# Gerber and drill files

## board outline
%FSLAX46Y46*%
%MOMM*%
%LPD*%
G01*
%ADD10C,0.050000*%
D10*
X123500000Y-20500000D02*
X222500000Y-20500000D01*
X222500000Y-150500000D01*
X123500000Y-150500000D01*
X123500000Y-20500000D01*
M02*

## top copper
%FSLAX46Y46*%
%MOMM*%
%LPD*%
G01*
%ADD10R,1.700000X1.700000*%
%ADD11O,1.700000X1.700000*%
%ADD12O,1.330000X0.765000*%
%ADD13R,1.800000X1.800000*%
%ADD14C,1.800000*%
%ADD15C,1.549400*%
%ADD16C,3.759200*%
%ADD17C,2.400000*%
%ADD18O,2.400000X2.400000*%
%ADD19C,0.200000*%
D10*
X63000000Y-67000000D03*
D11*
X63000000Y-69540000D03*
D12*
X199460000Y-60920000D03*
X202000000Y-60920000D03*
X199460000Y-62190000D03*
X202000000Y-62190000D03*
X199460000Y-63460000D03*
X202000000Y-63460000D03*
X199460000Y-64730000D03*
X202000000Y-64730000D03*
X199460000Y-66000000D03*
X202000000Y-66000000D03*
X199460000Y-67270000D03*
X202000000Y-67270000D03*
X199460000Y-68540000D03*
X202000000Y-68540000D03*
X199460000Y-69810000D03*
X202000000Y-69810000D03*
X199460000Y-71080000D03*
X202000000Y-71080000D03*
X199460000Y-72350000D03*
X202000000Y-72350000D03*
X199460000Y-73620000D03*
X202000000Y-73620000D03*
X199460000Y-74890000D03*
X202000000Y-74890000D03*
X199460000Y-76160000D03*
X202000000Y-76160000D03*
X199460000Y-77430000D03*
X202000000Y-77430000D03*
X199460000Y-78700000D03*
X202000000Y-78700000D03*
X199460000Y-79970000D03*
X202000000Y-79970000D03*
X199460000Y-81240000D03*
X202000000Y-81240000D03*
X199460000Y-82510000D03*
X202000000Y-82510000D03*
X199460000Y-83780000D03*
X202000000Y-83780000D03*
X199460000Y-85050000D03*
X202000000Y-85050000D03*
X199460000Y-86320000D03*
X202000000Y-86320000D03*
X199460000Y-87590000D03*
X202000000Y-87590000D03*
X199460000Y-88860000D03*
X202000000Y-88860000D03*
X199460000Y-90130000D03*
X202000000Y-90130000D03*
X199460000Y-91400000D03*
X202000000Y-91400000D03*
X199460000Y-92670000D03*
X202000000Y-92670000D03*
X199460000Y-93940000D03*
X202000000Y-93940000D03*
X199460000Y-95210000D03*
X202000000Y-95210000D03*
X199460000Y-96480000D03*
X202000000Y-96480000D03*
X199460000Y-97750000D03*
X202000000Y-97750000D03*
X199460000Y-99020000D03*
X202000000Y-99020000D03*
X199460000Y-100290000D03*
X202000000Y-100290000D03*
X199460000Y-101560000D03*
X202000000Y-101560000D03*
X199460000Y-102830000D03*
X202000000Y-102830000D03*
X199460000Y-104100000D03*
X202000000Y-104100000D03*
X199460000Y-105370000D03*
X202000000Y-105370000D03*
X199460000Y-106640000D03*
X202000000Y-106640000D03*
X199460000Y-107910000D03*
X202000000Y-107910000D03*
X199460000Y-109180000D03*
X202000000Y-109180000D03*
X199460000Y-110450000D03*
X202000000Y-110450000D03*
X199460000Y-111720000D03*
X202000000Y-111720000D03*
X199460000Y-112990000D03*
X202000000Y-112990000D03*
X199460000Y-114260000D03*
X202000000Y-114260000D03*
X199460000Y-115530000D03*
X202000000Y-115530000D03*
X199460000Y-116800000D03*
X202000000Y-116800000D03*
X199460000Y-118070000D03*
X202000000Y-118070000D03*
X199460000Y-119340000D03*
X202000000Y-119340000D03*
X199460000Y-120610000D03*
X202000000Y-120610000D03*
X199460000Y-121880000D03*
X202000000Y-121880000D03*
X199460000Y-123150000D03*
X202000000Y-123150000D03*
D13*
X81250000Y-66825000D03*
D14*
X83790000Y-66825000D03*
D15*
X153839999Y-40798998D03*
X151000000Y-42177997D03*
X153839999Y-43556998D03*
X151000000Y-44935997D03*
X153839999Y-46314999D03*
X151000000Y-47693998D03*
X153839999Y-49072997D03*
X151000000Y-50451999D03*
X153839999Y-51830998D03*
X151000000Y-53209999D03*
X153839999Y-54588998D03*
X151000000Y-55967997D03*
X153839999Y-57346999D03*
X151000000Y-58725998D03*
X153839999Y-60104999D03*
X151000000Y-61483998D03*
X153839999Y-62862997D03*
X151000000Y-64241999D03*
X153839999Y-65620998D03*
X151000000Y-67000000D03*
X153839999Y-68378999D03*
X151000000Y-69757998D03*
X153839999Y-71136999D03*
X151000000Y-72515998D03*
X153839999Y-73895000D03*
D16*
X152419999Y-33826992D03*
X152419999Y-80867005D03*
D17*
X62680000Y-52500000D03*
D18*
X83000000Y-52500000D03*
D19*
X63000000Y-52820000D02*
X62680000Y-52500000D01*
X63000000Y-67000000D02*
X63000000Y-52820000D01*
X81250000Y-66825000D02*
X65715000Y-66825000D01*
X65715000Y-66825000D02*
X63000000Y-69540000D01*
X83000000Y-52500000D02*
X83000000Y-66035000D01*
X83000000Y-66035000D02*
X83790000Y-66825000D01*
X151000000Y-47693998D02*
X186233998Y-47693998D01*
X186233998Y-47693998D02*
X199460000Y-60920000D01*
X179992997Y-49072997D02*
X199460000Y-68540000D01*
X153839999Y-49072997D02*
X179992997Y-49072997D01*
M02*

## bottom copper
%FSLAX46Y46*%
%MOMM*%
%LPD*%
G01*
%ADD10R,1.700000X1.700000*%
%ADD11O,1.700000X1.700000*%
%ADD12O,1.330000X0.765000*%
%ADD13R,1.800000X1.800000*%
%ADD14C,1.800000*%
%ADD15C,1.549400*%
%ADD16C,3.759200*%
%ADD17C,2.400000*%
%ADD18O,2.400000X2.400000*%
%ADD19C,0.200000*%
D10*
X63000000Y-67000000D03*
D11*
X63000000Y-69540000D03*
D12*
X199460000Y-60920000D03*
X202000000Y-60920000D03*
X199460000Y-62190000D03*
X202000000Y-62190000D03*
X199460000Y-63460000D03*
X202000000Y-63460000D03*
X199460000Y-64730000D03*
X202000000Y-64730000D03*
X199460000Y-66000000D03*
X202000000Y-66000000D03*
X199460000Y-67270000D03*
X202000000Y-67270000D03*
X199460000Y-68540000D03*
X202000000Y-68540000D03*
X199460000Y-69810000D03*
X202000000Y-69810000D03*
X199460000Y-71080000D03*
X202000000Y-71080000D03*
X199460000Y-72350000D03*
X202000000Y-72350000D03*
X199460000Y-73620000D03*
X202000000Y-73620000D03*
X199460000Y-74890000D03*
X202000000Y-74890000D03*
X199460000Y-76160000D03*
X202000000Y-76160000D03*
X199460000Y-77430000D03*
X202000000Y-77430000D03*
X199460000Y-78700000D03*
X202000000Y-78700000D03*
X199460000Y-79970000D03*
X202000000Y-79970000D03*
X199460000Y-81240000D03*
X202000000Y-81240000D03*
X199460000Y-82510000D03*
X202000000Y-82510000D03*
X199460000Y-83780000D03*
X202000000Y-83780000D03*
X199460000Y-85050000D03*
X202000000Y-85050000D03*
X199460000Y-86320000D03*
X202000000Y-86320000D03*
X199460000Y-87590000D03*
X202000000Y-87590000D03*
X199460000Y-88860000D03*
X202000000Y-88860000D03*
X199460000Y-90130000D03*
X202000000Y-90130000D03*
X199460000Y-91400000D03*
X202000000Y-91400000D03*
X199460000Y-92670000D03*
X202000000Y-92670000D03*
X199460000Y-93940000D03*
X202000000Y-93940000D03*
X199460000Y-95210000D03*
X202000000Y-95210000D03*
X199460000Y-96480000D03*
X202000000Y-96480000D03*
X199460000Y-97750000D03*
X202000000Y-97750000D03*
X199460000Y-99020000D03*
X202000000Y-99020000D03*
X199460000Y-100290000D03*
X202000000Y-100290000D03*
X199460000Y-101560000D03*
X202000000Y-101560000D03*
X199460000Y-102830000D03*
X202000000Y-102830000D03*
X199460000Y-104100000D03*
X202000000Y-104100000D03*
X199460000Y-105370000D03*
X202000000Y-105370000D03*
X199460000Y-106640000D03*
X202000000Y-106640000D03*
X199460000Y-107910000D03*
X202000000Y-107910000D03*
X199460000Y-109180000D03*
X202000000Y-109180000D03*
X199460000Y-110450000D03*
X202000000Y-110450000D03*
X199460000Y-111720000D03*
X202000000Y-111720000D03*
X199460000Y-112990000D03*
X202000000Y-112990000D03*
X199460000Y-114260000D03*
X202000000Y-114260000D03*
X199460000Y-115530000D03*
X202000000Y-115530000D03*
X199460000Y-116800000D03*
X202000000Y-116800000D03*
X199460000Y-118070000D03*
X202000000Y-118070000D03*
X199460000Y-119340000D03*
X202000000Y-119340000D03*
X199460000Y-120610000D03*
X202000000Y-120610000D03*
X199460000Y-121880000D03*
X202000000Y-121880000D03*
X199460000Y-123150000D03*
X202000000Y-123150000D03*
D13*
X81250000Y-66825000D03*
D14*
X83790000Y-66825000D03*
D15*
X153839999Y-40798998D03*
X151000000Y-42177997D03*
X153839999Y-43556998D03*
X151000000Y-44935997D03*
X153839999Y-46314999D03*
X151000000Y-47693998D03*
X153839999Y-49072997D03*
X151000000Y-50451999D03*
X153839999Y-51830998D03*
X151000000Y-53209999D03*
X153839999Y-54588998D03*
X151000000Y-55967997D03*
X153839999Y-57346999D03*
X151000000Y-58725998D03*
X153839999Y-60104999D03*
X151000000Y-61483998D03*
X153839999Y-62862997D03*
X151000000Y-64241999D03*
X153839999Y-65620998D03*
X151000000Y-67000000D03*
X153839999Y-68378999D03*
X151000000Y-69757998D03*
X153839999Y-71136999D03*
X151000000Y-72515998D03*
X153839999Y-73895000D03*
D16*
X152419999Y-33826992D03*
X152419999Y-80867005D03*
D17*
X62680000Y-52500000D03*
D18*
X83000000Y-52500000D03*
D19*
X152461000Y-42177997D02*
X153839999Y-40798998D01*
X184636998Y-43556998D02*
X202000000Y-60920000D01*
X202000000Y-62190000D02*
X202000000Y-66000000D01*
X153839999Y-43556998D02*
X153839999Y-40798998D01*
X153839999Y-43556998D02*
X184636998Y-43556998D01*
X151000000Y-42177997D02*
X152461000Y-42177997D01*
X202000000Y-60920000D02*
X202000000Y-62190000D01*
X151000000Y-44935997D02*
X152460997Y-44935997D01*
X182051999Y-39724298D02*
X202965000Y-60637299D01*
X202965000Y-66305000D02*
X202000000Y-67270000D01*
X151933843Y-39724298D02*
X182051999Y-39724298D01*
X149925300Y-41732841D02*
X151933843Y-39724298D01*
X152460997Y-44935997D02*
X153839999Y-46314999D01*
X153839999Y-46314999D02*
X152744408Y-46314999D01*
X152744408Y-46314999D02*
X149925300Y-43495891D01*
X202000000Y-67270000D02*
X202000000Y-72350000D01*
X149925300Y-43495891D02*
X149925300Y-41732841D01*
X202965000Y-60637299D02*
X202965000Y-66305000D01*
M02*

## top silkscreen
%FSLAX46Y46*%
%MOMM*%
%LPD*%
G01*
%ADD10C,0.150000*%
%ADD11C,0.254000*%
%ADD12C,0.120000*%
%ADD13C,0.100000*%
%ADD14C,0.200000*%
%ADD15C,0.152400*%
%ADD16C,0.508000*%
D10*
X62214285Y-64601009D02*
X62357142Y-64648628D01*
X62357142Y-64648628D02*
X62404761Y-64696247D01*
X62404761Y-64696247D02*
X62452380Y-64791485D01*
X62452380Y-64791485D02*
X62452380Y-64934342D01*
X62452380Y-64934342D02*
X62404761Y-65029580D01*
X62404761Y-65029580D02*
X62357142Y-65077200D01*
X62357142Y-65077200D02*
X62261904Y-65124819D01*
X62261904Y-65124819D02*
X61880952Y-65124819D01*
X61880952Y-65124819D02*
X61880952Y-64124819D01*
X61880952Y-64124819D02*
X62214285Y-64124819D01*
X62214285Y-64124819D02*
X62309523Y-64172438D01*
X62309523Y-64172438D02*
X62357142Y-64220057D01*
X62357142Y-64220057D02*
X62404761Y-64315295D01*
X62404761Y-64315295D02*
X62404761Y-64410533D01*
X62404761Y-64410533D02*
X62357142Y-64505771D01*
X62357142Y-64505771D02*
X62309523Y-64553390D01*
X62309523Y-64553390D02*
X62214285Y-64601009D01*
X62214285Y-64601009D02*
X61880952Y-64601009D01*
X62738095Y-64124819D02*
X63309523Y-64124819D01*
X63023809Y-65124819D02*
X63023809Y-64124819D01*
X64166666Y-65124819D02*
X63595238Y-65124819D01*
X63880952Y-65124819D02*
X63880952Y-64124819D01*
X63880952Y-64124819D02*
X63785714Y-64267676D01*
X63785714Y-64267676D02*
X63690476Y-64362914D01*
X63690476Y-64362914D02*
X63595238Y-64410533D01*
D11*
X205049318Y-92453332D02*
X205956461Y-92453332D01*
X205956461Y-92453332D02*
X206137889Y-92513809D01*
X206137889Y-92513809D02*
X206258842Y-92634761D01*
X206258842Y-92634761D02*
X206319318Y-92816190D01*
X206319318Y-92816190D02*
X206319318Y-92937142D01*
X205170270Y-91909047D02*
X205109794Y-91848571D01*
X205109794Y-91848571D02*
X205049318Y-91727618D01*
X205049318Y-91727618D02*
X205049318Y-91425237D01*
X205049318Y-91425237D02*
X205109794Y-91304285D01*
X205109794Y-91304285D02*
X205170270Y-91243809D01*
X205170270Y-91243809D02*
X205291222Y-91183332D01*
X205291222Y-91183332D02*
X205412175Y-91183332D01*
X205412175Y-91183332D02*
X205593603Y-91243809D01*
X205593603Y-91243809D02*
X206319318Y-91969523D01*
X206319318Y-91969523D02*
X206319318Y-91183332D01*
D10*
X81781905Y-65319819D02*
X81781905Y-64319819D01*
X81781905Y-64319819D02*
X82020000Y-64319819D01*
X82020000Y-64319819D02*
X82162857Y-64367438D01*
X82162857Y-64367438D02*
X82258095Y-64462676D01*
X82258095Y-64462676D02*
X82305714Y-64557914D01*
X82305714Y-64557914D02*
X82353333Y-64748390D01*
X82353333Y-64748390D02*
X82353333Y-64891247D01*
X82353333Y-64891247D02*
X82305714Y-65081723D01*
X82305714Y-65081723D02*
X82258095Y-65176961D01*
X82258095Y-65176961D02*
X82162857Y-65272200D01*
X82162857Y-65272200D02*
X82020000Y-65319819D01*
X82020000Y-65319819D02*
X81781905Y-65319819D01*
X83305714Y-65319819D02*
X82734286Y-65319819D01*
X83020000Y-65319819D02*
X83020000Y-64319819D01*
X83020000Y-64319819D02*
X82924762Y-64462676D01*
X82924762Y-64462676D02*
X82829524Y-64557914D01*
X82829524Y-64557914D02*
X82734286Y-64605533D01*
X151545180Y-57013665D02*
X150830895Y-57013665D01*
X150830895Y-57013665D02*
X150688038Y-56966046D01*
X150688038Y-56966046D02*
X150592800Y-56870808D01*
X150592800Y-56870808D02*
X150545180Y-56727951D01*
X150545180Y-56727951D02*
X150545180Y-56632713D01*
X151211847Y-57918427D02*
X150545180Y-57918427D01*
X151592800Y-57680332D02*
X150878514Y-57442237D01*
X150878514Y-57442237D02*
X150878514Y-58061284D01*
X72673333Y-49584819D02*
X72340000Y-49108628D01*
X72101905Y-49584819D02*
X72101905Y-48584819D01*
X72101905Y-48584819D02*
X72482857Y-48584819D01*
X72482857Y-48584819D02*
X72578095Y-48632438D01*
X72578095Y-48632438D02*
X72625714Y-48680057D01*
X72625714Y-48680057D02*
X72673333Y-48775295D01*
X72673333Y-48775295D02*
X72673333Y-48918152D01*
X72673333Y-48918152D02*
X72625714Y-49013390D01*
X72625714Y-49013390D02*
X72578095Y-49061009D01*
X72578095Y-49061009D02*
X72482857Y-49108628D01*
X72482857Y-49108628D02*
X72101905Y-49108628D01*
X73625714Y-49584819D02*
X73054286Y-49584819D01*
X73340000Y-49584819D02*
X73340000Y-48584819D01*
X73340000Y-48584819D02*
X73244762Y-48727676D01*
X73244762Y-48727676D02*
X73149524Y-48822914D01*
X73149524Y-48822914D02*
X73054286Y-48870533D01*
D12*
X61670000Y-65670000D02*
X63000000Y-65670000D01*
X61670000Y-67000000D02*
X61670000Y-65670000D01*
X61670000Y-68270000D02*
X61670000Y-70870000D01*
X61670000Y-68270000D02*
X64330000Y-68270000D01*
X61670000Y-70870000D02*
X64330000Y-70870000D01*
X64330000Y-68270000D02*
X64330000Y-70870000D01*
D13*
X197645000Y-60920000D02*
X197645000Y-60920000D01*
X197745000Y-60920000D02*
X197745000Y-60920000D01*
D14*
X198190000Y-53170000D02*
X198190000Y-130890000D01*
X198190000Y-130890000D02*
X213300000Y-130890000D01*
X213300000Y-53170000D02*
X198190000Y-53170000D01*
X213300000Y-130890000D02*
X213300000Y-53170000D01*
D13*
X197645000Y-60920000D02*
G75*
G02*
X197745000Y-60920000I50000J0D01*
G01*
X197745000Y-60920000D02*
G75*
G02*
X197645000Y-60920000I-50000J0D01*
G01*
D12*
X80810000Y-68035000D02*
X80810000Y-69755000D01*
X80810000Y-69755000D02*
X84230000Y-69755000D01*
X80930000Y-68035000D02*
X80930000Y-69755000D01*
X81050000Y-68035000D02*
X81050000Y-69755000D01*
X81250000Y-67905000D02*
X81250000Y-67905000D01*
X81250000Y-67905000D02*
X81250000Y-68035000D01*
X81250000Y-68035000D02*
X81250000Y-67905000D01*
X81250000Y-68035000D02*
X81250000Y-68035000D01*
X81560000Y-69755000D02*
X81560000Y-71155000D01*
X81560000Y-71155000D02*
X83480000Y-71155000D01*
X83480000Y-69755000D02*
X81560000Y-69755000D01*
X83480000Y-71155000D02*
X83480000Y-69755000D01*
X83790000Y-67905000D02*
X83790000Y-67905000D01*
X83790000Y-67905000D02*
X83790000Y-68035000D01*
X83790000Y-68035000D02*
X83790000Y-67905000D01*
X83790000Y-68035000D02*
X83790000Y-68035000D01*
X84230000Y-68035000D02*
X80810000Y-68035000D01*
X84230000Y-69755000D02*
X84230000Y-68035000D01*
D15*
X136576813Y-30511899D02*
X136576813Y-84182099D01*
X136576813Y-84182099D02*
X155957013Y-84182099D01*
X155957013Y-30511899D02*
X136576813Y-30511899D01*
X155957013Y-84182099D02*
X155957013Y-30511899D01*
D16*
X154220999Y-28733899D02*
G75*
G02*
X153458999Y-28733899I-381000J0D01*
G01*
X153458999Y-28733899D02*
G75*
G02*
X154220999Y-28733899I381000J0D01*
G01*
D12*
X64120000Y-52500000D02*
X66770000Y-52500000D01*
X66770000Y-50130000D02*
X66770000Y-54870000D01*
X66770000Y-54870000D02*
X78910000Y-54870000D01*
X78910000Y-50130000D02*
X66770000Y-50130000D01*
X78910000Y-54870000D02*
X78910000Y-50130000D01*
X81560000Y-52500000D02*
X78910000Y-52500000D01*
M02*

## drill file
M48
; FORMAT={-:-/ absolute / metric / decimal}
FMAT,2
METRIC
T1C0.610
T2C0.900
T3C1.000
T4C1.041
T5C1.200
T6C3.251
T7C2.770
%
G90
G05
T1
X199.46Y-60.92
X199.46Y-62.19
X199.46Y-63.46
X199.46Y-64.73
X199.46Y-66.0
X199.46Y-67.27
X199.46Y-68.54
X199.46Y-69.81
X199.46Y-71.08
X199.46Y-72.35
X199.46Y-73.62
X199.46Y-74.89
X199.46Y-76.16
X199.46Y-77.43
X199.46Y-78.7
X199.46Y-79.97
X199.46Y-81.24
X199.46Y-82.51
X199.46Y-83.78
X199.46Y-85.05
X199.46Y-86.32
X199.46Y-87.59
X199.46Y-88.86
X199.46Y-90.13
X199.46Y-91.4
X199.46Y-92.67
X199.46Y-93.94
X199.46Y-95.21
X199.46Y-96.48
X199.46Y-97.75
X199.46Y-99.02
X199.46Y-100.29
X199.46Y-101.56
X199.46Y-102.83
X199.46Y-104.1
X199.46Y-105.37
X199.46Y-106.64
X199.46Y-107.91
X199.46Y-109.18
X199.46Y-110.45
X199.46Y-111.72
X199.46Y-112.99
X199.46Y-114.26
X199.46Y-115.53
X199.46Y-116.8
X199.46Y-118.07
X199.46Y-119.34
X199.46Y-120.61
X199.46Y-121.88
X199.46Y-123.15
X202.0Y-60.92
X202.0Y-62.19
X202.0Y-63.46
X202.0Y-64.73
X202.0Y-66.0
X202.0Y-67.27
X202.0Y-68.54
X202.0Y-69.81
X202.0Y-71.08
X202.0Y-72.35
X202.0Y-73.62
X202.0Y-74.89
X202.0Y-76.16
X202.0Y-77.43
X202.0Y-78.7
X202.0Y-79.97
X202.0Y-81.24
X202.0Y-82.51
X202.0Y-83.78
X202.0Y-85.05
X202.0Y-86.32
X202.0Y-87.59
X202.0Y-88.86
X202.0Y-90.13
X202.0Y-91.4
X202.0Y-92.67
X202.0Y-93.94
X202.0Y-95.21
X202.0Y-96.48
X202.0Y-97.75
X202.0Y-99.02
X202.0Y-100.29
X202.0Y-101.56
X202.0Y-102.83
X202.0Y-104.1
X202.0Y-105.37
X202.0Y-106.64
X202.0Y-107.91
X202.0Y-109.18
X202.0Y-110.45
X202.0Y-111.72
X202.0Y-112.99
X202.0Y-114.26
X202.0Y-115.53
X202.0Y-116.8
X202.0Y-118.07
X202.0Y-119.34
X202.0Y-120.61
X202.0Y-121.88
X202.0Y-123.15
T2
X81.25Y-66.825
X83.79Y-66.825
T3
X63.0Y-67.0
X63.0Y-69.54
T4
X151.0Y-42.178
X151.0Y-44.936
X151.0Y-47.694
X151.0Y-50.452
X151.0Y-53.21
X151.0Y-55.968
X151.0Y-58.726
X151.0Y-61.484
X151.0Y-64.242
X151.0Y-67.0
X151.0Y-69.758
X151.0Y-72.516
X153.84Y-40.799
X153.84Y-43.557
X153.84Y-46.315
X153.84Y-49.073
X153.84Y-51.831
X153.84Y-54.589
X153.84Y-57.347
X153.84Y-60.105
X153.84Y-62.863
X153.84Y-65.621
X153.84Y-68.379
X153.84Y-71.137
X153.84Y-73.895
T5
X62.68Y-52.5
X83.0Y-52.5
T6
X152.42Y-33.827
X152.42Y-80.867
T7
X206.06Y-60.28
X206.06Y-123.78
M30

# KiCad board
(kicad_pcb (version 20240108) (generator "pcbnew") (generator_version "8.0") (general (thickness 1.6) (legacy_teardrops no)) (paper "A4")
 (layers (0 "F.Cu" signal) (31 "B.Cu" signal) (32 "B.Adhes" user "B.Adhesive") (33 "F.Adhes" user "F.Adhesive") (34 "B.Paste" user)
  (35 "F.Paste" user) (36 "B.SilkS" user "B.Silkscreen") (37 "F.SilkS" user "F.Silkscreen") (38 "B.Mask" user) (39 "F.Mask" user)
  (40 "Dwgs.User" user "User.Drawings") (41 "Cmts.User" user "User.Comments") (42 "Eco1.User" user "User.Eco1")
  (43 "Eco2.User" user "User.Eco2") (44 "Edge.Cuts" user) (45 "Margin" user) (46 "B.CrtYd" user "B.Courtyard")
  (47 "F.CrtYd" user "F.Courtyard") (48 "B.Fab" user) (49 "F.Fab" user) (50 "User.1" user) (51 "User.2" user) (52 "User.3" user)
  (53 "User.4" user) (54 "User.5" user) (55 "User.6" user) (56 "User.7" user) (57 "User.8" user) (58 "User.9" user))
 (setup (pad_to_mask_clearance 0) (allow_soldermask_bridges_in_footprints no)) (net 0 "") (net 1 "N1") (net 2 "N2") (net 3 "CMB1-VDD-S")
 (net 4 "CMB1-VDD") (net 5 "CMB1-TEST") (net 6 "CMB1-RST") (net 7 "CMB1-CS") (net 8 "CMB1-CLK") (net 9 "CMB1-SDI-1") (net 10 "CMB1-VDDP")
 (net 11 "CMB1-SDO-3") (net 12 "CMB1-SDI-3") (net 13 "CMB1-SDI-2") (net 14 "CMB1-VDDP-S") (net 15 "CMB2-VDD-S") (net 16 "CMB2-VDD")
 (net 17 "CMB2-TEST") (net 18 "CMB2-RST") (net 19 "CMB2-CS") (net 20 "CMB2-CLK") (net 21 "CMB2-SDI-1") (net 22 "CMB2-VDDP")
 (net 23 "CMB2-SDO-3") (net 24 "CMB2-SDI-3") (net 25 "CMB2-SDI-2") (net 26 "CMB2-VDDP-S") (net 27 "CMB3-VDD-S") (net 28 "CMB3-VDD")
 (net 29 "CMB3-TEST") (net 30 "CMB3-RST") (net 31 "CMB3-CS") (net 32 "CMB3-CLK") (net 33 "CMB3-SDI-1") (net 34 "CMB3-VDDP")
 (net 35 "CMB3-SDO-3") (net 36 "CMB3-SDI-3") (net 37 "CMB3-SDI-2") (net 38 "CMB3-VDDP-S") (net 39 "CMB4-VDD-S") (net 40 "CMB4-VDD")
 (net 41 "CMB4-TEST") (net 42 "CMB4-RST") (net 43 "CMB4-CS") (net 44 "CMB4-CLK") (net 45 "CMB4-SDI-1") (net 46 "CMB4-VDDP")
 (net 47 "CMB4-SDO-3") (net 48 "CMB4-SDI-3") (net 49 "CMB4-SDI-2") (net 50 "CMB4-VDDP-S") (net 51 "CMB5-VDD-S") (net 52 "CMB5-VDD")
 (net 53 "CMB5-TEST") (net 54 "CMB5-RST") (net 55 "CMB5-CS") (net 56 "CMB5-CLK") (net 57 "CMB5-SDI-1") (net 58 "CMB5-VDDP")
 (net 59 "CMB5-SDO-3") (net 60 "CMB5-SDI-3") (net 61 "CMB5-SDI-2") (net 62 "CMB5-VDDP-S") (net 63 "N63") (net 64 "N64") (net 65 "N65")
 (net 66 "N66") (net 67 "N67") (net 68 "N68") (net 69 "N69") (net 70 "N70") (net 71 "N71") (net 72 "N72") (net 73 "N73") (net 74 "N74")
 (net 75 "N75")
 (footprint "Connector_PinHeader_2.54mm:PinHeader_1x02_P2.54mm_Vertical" (layer "F.Cu") (at 63 67)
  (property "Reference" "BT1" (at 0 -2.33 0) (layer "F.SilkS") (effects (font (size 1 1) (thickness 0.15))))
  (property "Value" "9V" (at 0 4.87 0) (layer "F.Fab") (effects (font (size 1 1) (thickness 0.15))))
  (fp_line (start -1.33 -1.33) (end 0 -1.33) (stroke (width 0.12) (type solid)) (layer "F.SilkS"))
  (fp_line (start -1.33 0) (end -1.33 -1.33) (stroke (width 0.12) (type solid)) (layer "F.SilkS"))
  (fp_line (start -1.33 1.27) (end -1.33 3.87) (stroke (width 0.12) (type solid)) (layer "F.SilkS"))
  (fp_line (start -1.33 1.27) (end 1.33 1.27) (stroke (width 0.12) (type solid)) (layer "F.SilkS"))
  (fp_line (start -1.33 3.87) (end 1.33 3.87) (stroke (width 0.12) (type solid)) (layer "F.SilkS"))
  (fp_line (start 1.33 1.27) (end 1.33 3.87) (stroke (width 0.12) (type solid)) (layer "F.SilkS"))
  (pad "1" thru_hole rect (at 0 0) (size 1.7 1.7) (drill 1) (layers "*.Cu" "*.Mask") (remove_unused_layers no) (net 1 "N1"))
  (pad "2" thru_hole oval (at 0 2.54) (size 1.7 1.7) (drill 1) (layers "*.Cu" "*.Mask") (remove_unused_layers no) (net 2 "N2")))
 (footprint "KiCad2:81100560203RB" (layer "F.Cu") (at 199.46 60.92 -90)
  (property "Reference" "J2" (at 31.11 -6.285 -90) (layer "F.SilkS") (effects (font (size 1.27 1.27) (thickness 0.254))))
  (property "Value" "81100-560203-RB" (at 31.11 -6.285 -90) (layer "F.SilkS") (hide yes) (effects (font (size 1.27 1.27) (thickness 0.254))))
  (fp_line (start 0 1.815) (end 0 1.815) (stroke (width 0.1) (type solid)) (layer "F.SilkS"))
  (fp_line (start 0 1.715) (end 0 1.715) (stroke (width 0.1) (type solid)) (layer "F.SilkS"))
  (fp_line (start -7.75 1.27) (end 69.97 1.27) (stroke (width 0.2) (type solid)) (layer "F.SilkS"))
  (fp_line (start 69.97 1.27) (end 69.97 -13.84) (stroke (width 0.2) (type solid)) (layer "F.SilkS"))
  (fp_line (start -7.75 -13.84) (end -7.75 1.27) (stroke (width 0.2) (type solid)) (layer "F.SilkS"))
  (fp_line (start 69.97 -13.84) (end -7.75 -13.84) (stroke (width 0.2) (type solid)) (layer "F.SilkS"))
  (fp_arc (start 0 1.815) (mid -0.05 1.765) (end 0 1.715) (stroke (width 0.1) (type solid)) (layer "F.SilkS"))
  (fp_arc (start 0 1.715) (mid 0.05 1.765) (end 0 1.815) (stroke (width 0.1) (type solid)) (layer "F.SilkS"))
  (pad "" np_thru_hole circle (at -0.64 -6.6 270) (size 2.77 2.77) (drill 2.77) (layers "*.Cu" "*.Mask"))
  (pad "" np_thru_hole circle (at 62.86 -6.6 270) (size 2.77 2.77) (drill 2.77) (layers "*.Cu" "*.Mask"))
  (pad "1" thru_hole oval (at 0 0 270) (size 0.765 1.33) (drill 0.61) (layers "*.Cu" "*.Mask") (remove_unused_layers no)
   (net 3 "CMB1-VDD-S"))
  (pad "2" thru_hole oval (at 0 -2.54 270) (size 0.765 1.33) (drill 0.61) (layers "*.Cu" "*.Mask") (remove_unused_layers no)
   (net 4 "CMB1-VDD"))
  (pad "3" thru_hole oval (at 1.27 0 270) (size 0.765 1.33) (drill 0.61) (layers "*.Cu" "*.Mask") (remove_unused_layers no)
   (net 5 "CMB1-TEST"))
  (pad "4" thru_hole oval (at 1.27 -2.54 270) (size 0.765 1.33) (drill 0.61) (layers "*.Cu" "*.Mask") (remove_unused_layers no)
   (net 4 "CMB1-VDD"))
  (pad "5" thru_hole oval (at 2.54 0 270) (size 0.765 1.33) (drill 0.61) (layers "*.Cu" "*.Mask") (remove_unused_layers no)
   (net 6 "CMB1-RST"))
  (pad "6" thru_hole oval (at 2.54 -2.54 270) (size 0.765 1.33) (drill 0.61) (layers "*.Cu" "*.Mask") (remove_unused_layers no)
   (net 4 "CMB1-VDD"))
  (pad "7" thru_hole oval (at 3.81 0 270) (size 0.765 1.33) (drill 0.61) (layers "*.Cu" "*.Mask") (remove_unused_layers no)
   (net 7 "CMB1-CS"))
  (pad "8" thru_hole oval (at 3.81 -2.54 270) (size 0.765 1.33) (drill 0.61) (layers "*.Cu" "*.Mask") (remove_unused_layers no)
   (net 4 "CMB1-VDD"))
  (pad "9" thru_hole oval (at 5.08 0 270) (size 0.765 1.33) (drill 0.61) (layers "*.Cu" "*.Mask") (remove_unused_layers no)
   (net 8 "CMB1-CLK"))
  (pad "10" thru_hole oval (at 5.08 -2.54 270) (size 0.765 1.33) (drill 0.61) (layers "*.Cu" "*.Mask") (remove_unused_layers no)
   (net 4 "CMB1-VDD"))
  (pad "11" thru_hole oval (at 6.35 0 270) (size 0.765 1.33) (drill 0.61) (layers "*.Cu" "*.Mask") (remove_unused_layers no)
   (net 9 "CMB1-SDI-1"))
  (pad "12" thru_hole oval (at 6.35 -2.54 270) (size 0.765 1.33) (drill 0.61) (layers "*.Cu" "*.Mask") (remove_unused_layers no)
   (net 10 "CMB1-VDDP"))
  (pad "13" thru_hole oval (at 7.62 0 270) (size 0.765 1.33) (drill 0.61) (layers "*.Cu" "*.Mask") (remove_unused_layers no)
   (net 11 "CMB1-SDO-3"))
  (pad "14" thru_hole oval (at 7.62 -2.54 270) (size 0.765 1.33) (drill 0.61) (layers "*.Cu" "*.Mask") (remove_unused_layers no)
   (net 10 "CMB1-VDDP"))
  (pad "15" thru_hole oval (at 8.89 0 270) (size 0.765 1.33) (drill 0.61) (layers "*.Cu" "*.Mask") (remove_unused_layers no)
   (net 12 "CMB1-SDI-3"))
  (pad "16" thru_hole oval (at 8.89 -2.54 270) (size 0.765 1.33) (drill 0.61) (layers "*.Cu" "*.Mask") (remove_unused_layers no)
   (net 10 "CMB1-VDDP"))
  (pad "17" thru_hole oval (at 10.16 0 270) (size 0.765 1.33) (drill 0.61) (layers "*.Cu" "*.Mask") (remove_unused_layers no)
   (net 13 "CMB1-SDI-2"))
  (pad "18" thru_hole oval (at 10.16 -2.54 270) (size 0.765 1.33) (drill 0.61) (layers "*.Cu" "*.Mask") (remove_unused_layers no)
   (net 10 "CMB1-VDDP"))
  (pad "19" thru_hole oval (at 11.43 0 270) (size 0.765 1.33) (drill 0.61) (layers "*.Cu" "*.Mask") (remove_unused_layers no)
   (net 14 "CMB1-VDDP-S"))
  (pad "20" thru_hole oval (at 11.43 -2.54 270) (size 0.765 1.33) (drill 0.61) (layers "*.Cu" "*.Mask") (remove_unused_layers no)
   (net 10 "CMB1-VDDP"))
  (pad "21" thru_hole oval (at 12.7 0 270) (size 0.765 1.33) (drill 0.61) (layers "*.Cu" "*.Mask") (remove_unused_layers no)
   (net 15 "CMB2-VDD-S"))
  (pad "22" thru_hole oval (at 12.7 -2.54 270) (size 0.765 1.33) (drill 0.61) (layers "*.Cu" "*.Mask") (remove_unused_layers no)
   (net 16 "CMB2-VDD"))
  (pad "23" thru_hole oval (at 13.97 0 270) (size 0.765 1.33) (drill 0.61) (layers "*.Cu" "*.Mask") (remove_unused_layers no)
   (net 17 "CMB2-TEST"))
  (pad "24" thru_hole oval (at 13.97 -2.54 270) (size 0.765 1.33) (drill 0.61) (layers "*.Cu" "*.Mask") (remove_unused_layers no)
   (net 16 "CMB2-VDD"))
  (pad "25" thru_hole oval (at 15.24 0 270) (size 0.765 1.33) (drill 0.61) (layers "*.Cu" "*.Mask") (remove_unused_layers no)
   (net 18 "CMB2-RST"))
  (pad "26" thru_hole oval (at 15.24 -2.54 270) (size 0.765 1.33) (drill 0.61) (layers "*.Cu" "*.Mask") (remove_unused_layers no)
   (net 16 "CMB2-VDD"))
  (pad "27" thru_hole oval (at 16.51 0 270) (size 0.765 1.33) (drill 0.61) (layers "*.Cu" "*.Mask") (remove_unused_layers no)
   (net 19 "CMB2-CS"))
  (pad "28" thru_hole oval (at 16.51 -2.54 270) (size 0.765 1.33) (drill 0.61) (layers "*.Cu" "*.Mask") (remove_unused_layers no)
   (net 16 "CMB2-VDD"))
  (pad "29" thru_hole oval (at 17.78 0 270) (size 0.765 1.33) (drill 0.61) (layers "*.Cu" "*.Mask") (remove_unused_layers no)
   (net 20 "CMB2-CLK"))
  (pad "30" thru_hole oval (at 17.78 -2.54 270) (size 0.765 1.33) (drill 0.61) (layers "*.Cu" "*.Mask") (remove_unused_layers no)
   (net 16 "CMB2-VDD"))
  (pad "31" thru_hole oval (at 19.05 0 270) (size 0.765 1.33) (drill 0.61) (layers "*.Cu" "*.Mask") (remove_unused_layers no)
   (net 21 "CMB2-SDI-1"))
  (pad "32" thru_hole oval (at 19.05 -2.54 270) (size 0.765 1.33) (drill 0.61) (layers "*.Cu" "*.Mask") (remove_unused_layers no)
   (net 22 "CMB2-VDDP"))
  (pad "33" thru_hole oval (at 20.32 0 270) (size 0.765 1.33) (drill 0.61) (layers "*.Cu" "*.Mask") (remove_unused_layers no)
   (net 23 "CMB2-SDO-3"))
  (pad "34" thru_hole oval (at 20.32 -2.54 270) (size 0.765 1.33) (drill 0.61) (layers "*.Cu" "*.Mask") (remove_unused_layers no)
   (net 22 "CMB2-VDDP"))
  (pad "35" thru_hole oval (at 21.59 0 270) (size 0.765 1.33) (drill 0.61) (layers "*.Cu" "*.Mask") (remove_unused_layers no)
   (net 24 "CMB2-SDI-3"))
  (pad "36" thru_hole oval (at 21.59 -2.54 270) (size 0.765 1.33) (drill 0.61) (layers "*.Cu" "*.Mask") (remove_unused_layers no)
   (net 22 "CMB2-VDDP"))
  (pad "37" thru_hole oval (at 22.86 0 270) (size 0.765 1.33) (drill 0.61) (layers "*.Cu" "*.Mask") (remove_unused_layers no)
   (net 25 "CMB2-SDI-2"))
  (pad "38" thru_hole oval (at 22.86 -2.54 270) (size 0.765 1.33) (drill 0.61) (layers "*.Cu" "*.Mask") (remove_unused_layers no)
   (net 22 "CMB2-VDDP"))
  (pad "39" thru_hole oval (at 24.13 0 270) (size 0.765 1.33) (drill 0.61) (layers "*.Cu" "*.Mask") (remove_unused_layers no)
   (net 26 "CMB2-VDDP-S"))
  (pad "40" thru_hole oval (at 24.13 -2.54 270) (size 0.765 1.33) (drill 0.61) (layers "*.Cu" "*.Mask") (remove_unused_layers no)
   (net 22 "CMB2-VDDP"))
  (pad "41" thru_hole oval (at 25.4 0 270) (size 0.765 1.33) (drill 0.61) (layers "*.Cu" "*.Mask") (remove_unused_layers no)
   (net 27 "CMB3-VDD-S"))
  (pad "42" thru_hole oval (at 25.4 -2.54 270) (size 0.765 1.33) (drill 0.61) (layers "*.Cu" "*.Mask") (remove_unused_layers no)
   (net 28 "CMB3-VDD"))
  (pad "43" thru_hole oval (at 26.67 0 270) (size 0.765 1.33) (drill 0.61) (layers "*.Cu" "*.Mask") (remove_unused_layers no)
   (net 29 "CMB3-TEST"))
  (pad "44" thru_hole oval (at 26.67 -2.54 270) (size 0.765 1.33) (drill 0.61) (layers "*.Cu" "*.Mask") (remove_unused_layers no)
   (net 28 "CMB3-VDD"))
  (pad "45" thru_hole oval (at 27.94 0 270) (size 0.765 1.33) (drill 0.61) (layers "*.Cu" "*.Mask") (remove_unused_layers no)
   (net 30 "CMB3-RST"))
  (pad "46" thru_hole oval (at 27.94 -2.54 270) (size 0.765 1.33) (drill 0.61) (layers "*.Cu" "*.Mask") (remove_unused_layers no)
   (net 28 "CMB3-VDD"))
  (pad "47" thru_hole oval (at 29.21 0 270) (size 0.765 1.33) (drill 0.61) (layers "*.Cu" "*.Mask") (remove_unused_layers no)
   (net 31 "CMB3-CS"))
  (pad "48" thru_hole oval (at 29.21 -2.54 270) (size 0.765 1.33) (drill 0.61) (layers "*.Cu" "*.Mask") (remove_unused_layers no)
   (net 28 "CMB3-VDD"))
  (pad "49" thru_hole oval (at 30.48 0 270) (size 0.765 1.33) (drill 0.61) (layers "*.Cu" "*.Mask") (remove_unused_layers no)
   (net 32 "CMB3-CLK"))
  (pad "50" thru_hole oval (at 30.48 -2.54 270) (size 0.765 1.33) (drill 0.61) (layers "*.Cu" "*.Mask") (remove_unused_layers no)
   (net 28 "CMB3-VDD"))
  (pad "51" thru_hole oval (at 31.75 0 270) (size 0.765 1.33) (drill 0.61) (layers "*.Cu" "*.Mask") (remove_unused_layers no)
   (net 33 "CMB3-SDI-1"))
  (pad "52" thru_hole oval (at 31.75 -2.54 270) (size 0.765 1.33) (drill 0.61) (layers "*.Cu" "*.Mask") (remove_unused_layers no)
   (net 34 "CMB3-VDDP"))
  (pad "53" thru_hole oval (at 33.02 0 270) (size 0.765 1.33) (drill 0.61) (layers "*.Cu" "*.Mask") (remove_unused_layers no)
   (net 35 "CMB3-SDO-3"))
  (pad "54" thru_hole oval (at 33.02 -2.54 270) (size 0.765 1.33) (drill 0.61) (layers "*.Cu" "*.Mask") (remove_unused_layers no)
   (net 34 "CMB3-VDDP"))
  (pad "55" thru_hole oval (at 34.29 0 270) (size 0.765 1.33) (drill 0.61) (layers "*.Cu" "*.Mask") (remove_unused_layers no)
   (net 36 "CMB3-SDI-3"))
  (pad "56" thru_hole oval (at 34.29 -2.54 270) (size 0.765 1.33) (drill 0.61) (layers "*.Cu" "*.Mask") (remove_unused_layers no)
   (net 34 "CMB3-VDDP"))
  (pad "57" thru_hole oval (at 35.56 0 270) (size 0.765 1.33) (drill 0.61) (layers "*.Cu" "*.Mask") (remove_unused_layers no)
   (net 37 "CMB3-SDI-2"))
  (pad "58" thru_hole oval (at 35.56 -2.54 270) (size 0.765 1.33) (drill 0.61) (layers "*.Cu" "*.Mask") (remove_unused_layers no)
   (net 34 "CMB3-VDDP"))
  (pad "59" thru_hole oval (at 36.83 0 270) (size 0.765 1.33) (drill 0.61) (layers "*.Cu" "*.Mask") (remove_unused_layers no)
   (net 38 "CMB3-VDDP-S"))
  (pad "60" thru_hole oval (at 36.83 -2.54 270) (size 0.765 1.33) (drill 0.61) (layers "*.Cu" "*.Mask") (remove_unused_layers no)
   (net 34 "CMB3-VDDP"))
  (pad "61" thru_hole oval (at 38.1 0 270) (size 0.765 1.33) (drill 0.61) (layers "*.Cu" "*.Mask") (remove_unused_layers no)
   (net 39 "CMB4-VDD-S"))
  (pad "62" thru_hole oval (at 38.1 -2.54 270) (size 0.765 1.33) (drill 0.61) (layers "*.Cu" "*.Mask") (remove_unused_layers no)
   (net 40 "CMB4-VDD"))
  (pad "63" thru_hole oval (at 39.37 0 270) (size 0.765 1.33) (drill 0.61) (layers "*.Cu" "*.Mask") (remove_unused_layers no)
   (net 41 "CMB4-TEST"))
  (pad "64" thru_hole oval (at 39.37 -2.54 270) (size 0.765 1.33) (drill 0.61) (layers "*.Cu" "*.Mask") (remove_unused_layers no)
   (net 40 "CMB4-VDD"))
  (pad "65" thru_hole oval (at 40.64 0 270) (size 0.765 1.33) (drill 0.61) (layers "*.Cu" "*.Mask") (remove_unused_layers no)
   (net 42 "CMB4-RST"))
  (pad "66" thru_hole oval (at 40.64 -2.54 270) (size 0.765 1.33) (drill 0.61) (layers "*.Cu" "*.Mask") (remove_unused_layers no)
   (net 40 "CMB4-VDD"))
  (pad "67" thru_hole oval (at 41.91 0 270) (size 0.765 1.33) (drill 0.61) (layers "*.Cu" "*.Mask") (remove_unused_layers no)
   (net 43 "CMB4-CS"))
  (pad "68" thru_hole oval (at 41.91 -2.54 270) (size 0.765 1.33) (drill 0.61) (layers "*.Cu" "*.Mask") (remove_unused_layers no)
   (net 40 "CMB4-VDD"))
  (pad "69" thru_hole oval (at 43.18 0 270) (size 0.765 1.33) (drill 0.61) (layers "*.Cu" "*.Mask") (remove_unused_layers no)
   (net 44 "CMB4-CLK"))
  (pad "70" thru_hole oval (at 43.18 -2.54 270) (size 0.765 1.33) (drill 0.61) (layers "*.Cu" "*.Mask") (remove_unused_layers no)
   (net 40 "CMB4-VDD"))
  (pad "71" thru_hole oval (at 44.45 0 270) (size 0.765 1.33) (drill 0.61) (layers "*.Cu" "*.Mask") (remove_unused_layers no)
   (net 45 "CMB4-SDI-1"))
  (pad "72" thru_hole oval (at 44.45 -2.54 270) (size 0.765 1.33) (drill 0.61) (layers "*.Cu" "*.Mask") (remove_unused_layers no)
   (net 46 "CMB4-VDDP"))
  (pad "73" thru_hole oval (at 45.72 0 270) (size 0.765 1.33) (drill 0.61) (layers "*.Cu" "*.Mask") (remove_unused_layers no)
   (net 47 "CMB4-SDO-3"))
  (pad "74" thru_hole oval (at 45.72 -2.54 270) (size 0.765 1.33) (drill 0.61) (layers "*.Cu" "*.Mask") (remove_unused_layers no)
   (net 46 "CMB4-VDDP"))
  (pad "75" thru_hole oval (at 46.99 0 270) (size 0.765 1.33) (drill 0.61) (layers "*.Cu" "*.Mask") (remove_unused_layers no)
   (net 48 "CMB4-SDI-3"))
  (pad "76" thru_hole oval (at 46.99 -2.54 270) (size 0.765 1.33) (drill 0.61) (layers "*.Cu" "*.Mask") (remove_unused_layers no)
   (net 46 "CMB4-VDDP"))
  (pad "77" thru_hole oval (at 48.26 0 270) (size 0.765 1.33) (drill 0.61) (layers "*.Cu" "*.Mask") (remove_unused_layers no)
   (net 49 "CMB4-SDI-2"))
  (pad "78" thru_hole oval (at 48.26 -2.54 270) (size 0.765 1.33) (drill 0.61) (layers "*.Cu" "*.Mask") (remove_unused_layers no)
   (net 46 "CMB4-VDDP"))
  (pad "79" thru_hole oval (at 49.53 0 270) (size 0.765 1.33) (drill 0.61) (layers "*.Cu" "*.Mask") (remove_unused_layers no)
   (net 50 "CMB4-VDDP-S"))
  (pad "80" thru_hole oval (at 49.53 -2.54 270) (size 0.765 1.33) (drill 0.61) (layers "*.Cu" "*.Mask") (remove_unused_layers no)
   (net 46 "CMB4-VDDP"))
  (pad "81" thru_hole oval (at 50.8 0 270) (size 0.765 1.33) (drill 0.61) (layers "*.Cu" "*.Mask") (remove_unused_layers no)
   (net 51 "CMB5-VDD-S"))
  (pad "82" thru_hole oval (at 50.8 -2.54 270) (size 0.765 1.33) (drill 0.61) (layers "*.Cu" "*.Mask") (remove_unused_layers no)
   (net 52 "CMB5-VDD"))
  (pad "83" thru_hole oval (at 52.07 0 270) (size 0.765 1.33) (drill 0.61) (layers "*.Cu" "*.Mask") (remove_unused_layers no)
   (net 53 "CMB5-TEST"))
  (pad "84" thru_hole oval (at 52.07 -2.54 270) (size 0.765 1.33) (drill 0.61) (layers "*.Cu" "*.Mask") (remove_unused_layers no)
   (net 52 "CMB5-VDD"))
  (pad "85" thru_hole oval (at 53.34 0 270) (size 0.765 1.33) (drill 0.61) (layers "*.Cu" "*.Mask") (remove_unused_layers no)
   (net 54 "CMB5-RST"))
  (pad "86" thru_hole oval (at 53.34 -2.54 270) (size 0.765 1.33) (drill 0.61) (layers "*.Cu" "*.Mask") (remove_unused_layers no)
   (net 52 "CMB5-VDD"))
  (pad "87" thru_hole oval (at 54.61 0 270) (size 0.765 1.33) (drill 0.61) (layers "*.Cu" "*.Mask") (remove_unused_layers no)
   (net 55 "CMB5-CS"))
  (pad "88" thru_hole oval (at 54.61 -2.54 270) (size 0.765 1.33) (drill 0.61) (layers "*.Cu" "*.Mask") (remove_unused_layers no)
   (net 52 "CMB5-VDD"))
  (pad "89" thru_hole oval (at 55.88 0 270) (size 0.765 1.33) (drill 0.61) (layers "*.Cu" "*.Mask") (remove_unused_layers no)
   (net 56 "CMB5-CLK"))
  (pad "90" thru_hole oval (at 55.88 -2.54 270) (size 0.765 1.33) (drill 0.61) (layers "*.Cu" "*.Mask") (remove_unused_layers no)
   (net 52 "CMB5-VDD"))
  (pad "91" thru_hole oval (at 57.15 0 270) (size 0.765 1.33) (drill 0.61) (layers "*.Cu" "*.Mask") (remove_unused_layers no)
   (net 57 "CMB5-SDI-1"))
  (pad "92" thru_hole oval (at 57.15 -2.54 270) (size 0.765 1.33) (drill 0.61) (layers "*.Cu" "*.Mask") (remove_unused_layers no)
   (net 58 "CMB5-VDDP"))
  (pad "93" thru_hole oval (at 58.42 0 270) (size 0.765 1.33) (drill 0.61) (layers "*.Cu" "*.Mask") (remove_unused_layers no)
   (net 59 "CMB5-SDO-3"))
  (pad "94" thru_hole oval (at 58.42 -2.54 270) (size 0.765 1.33) (drill 0.61) (layers "*.Cu" "*.Mask") (remove_unused_layers no)
   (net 58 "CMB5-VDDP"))
  (pad "95" thru_hole oval (at 59.69 0 270) (size 0.765 1.33) (drill 0.61) (layers "*.Cu" "*.Mask") (remove_unused_layers no)
   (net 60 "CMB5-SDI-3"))
  (pad "96" thru_hole oval (at 59.69 -2.54 270) (size 0.765 1.33) (drill 0.61) (layers "*.Cu" "*.Mask") (remove_unused_layers no)
   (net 58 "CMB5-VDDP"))
  (pad "97" thru_hole oval (at 60.96 0 270) (size 0.765 1.33) (drill 0.61) (layers "*.Cu" "*.Mask") (remove_unused_layers no)
   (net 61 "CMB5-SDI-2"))
  (pad "98" thru_hole oval (at 60.96 -2.54 270) (size 0.765 1.33) (drill 0.61) (layers "*.Cu" "*.Mask") (remove_unused_layers no)
   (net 58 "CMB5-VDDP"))
  (pad "99" thru_hole oval (at 62.23 0 270) (size 0.765 1.33) (drill 0.61) (layers "*.Cu" "*.Mask") (remove_unused_layers no)
   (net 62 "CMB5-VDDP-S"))
  (pad "100" thru_hole oval (at 62.23 -2.54 270) (size 0.765 1.33) (drill 0.61) (layers "*.Cu" "*.Mask") (remove_unused_layers no)
   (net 58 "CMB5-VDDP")))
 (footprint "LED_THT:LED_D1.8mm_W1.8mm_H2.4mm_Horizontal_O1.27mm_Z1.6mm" (layer "F.Cu") (at 81.25 66.825)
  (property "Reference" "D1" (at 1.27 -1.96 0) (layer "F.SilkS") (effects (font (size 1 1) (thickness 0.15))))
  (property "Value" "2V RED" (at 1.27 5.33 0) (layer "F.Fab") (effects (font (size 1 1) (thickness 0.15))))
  (fp_line (start -0.44 1.21) (end -0.44 2.93) (stroke (width 0.12) (type solid)) (layer "F.SilkS"))
  (fp_line (start -0.44 2.93) (end 2.98 2.93) (stroke (width 0.12) (type solid)) (layer "F.SilkS"))
  (fp_line (start -0.32 1.21) (end -0.32 2.93) (stroke (width 0.12) (type solid)) (layer "F.SilkS"))
  (fp_line (start -0.2 1.21) (end -0.2 2.93) (stroke (width 0.12) (type solid)) (layer "F.SilkS"))
  (fp_line (start 0 1.08) (end 0 1.08) (stroke (width 0.12) (type solid)) (layer "F.SilkS"))
  (fp_line (start 0 1.08) (end 0 1.21) (stroke (width 0.12) (type solid)) (layer "F.SilkS"))
  (fp_line (start 0 1.21) (end 0 1.08) (stroke (width 0.12) (type solid)) (layer "F.SilkS"))
  (fp_line (start 0 1.21) (end 0 1.21) (stroke (width 0.12) (type solid)) (layer "F.SilkS"))
  (fp_line (start 0.31 2.93) (end 0.31 4.33) (stroke (width 0.12) (type solid)) (layer "F.SilkS"))
  (fp_line (start 0.31 4.33) (end 2.23 4.33) (stroke (width 0.12) (type solid)) (layer "F.SilkS"))
  (fp_line (start 2.23 2.93) (end 0.31 2.93) (stroke (width 0.12) (type solid)) (layer "F.SilkS"))
  (fp_line (start 2.23 4.33) (end 2.23 2.93) (stroke (width 0.12) (type solid)) (layer "F.SilkS"))
  (fp_line (start 2.54 1.08) (end 2.54 1.08) (stroke (width 0.12) (type solid)) (layer "F.SilkS"))
  (fp_line (start 2.54 1.08) (end 2.54 1.21) (stroke (width 0.12) (type solid)) (layer "F.SilkS"))
  (fp_line (start 2.54 1.21) (end 2.54 1.08) (stroke (width 0.12) (type solid)) (layer "F.SilkS"))
  (fp_line (start 2.54 1.21) (end 2.54 1.21) (stroke (width 0.12) (type solid)) (layer "F.SilkS"))
  (fp_line (start 2.98 1.21) (end -0.44 1.21) (stroke (width 0.12) (type solid)) (layer "F.SilkS"))
  (fp_line (start 2.98 2.93) (end 2.98 1.21) (stroke (width 0.12) (type solid)) (layer "F.SilkS"))
  (pad "1" thru_hole rect (at 0 0) (size 1.8 1.8) (drill 0.9) (layers "*.Cu" "*.Mask") (remove_unused_layers no) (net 2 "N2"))
  (pad "2" thru_hole circle (at 2.54 0) (size 1.8 1.8) (drill 0.9) (layers "*.Cu" "*.Mask") (remove_unused_layers no) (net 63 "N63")))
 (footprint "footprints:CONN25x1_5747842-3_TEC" (layer "F.Cu") (at 153.839999 40.798998 -90)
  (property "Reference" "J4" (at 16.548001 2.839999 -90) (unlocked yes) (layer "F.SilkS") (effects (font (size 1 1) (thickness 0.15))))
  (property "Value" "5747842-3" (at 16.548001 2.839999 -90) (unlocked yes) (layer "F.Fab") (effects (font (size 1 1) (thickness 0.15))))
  (fp_line (start -10.287099 17.263186) (end 43.383101 17.263186) (stroke (width 0.1524) (type solid)) (layer "F.SilkS"))
  (fp_line (start 43.383101 17.263186) (end 43.383101 -2.117014) (stroke (width 0.1524) (type solid)) (layer "F.SilkS"))
  (fp_line (start -10.287099 -2.117014) (end -10.287099 17.263186) (stroke (width 0.1524) (type solid)) (layer "F.SilkS"))
  (fp_line (start 43.383101 -2.117014) (end -10.287099 -2.117014) (stroke (width 0.1524) (type solid)) (layer "F.SilkS"))
  (fp_circle (center -12.065099 0) (end -11.684099 0) (stroke (width 0.508) (type solid)) (fill none) (layer "F.SilkS"))
  (pad "1" thru_hole circle (at 0 0 270) (size 1.5494 1.5494) (drill 1.0414) (layers "*.Cu" "*.Mask") (remove_unused_layers no)
   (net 4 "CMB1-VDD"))
  (pad "2" thru_hole circle (at 1.378999 2.839999 270) (size 1.5494 1.5494) (drill 1.0414) (layers "*.Cu" "*.Mask")
   (remove_unused_layers no) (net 4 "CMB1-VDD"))
  (pad "3" thru_hole circle (at 2.758 0 270) (size 1.5494 1.5494) (drill 1.0414) (layers "*.Cu" "*.Mask") (remove_unused_layers no)
   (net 4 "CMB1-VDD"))
  (pad "4" thru_hole circle (at 4.136999 2.839999 270) (size 1.5494 1.5494) (drill 1.0414) (layers "*.Cu" "*.Mask")
   (remove_unused_layers no) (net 10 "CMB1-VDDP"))
  (pad "5" thru_hole circle (at 5.516001 0 270) (size 1.5494 1.5494) (drill 1.0414) (layers "*.Cu" "*.Mask") (remove_unused_layers no)
   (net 10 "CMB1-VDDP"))
  (pad "6" thru_hole circle (at 6.895 2.839999 270) (size 1.5494 1.5494) (drill 1.0414) (layers "*.Cu" "*.Mask") (remove_unused_layers no)
   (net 3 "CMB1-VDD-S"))
  (pad "7" thru_hole circle (at 8.273999 0 270) (size 1.5494 1.5494) (drill 1.0414) (layers "*.Cu" "*.Mask") (remove_unused_layers no)
   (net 11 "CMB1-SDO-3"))
  (pad "8" thru_hole circle (at 9.653001 2.839999 270) (size 1.5494 1.5494) (drill 1.0414) (layers "*.Cu" "*.Mask")
   (remove_unused_layers no) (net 9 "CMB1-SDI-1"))
  (pad "9" thru_hole circle (at 11.032 0 270) (size 1.5494 1.5494) (drill 1.0414) (layers "*.Cu" "*.Mask") (remove_unused_layers no)
   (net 14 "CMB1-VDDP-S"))
  (pad "10" thru_hole circle (at 12.411001 2.839999 270) (size 1.5494 1.5494) (drill 1.0414) (layers "*.Cu" "*.Mask")
   (remove_unused_layers no) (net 15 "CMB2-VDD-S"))
  (pad "11" thru_hole circle (at 13.79 0 270) (size 1.5494 1.5494) (drill 1.0414) (layers "*.Cu" "*.Mask") (remove_unused_layers no)
   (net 23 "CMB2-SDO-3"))
  (pad "12" thru_hole circle (at 15.168999 2.839999 270) (size 1.5494 1.5494) (drill 1.0414) (layers "*.Cu" "*.Mask")
   (remove_unused_layers no) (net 21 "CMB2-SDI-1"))
  (pad "13" thru_hole circle (at 16.548001 0 270) (size 1.5494 1.5494) (drill 1.0414) (layers "*.Cu" "*.Mask") (remove_unused_layers no)
   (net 26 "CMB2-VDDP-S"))
  (pad "14" thru_hole circle (at 17.927 2.839999 270) (size 1.5494 1.5494) (drill 1.0414) (layers "*.Cu" "*.Mask") (remove_unused_layers no)
   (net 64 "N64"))
  (pad "15" thru_hole circle (at 19.306001 0 270) (size 1.5494 1.5494) (drill 1.0414) (layers "*.Cu" "*.Mask") (remove_unused_layers no)
   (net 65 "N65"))
  (pad "16" thru_hole circle (at 20.685 2.839999 270) (size 1.5494 1.5494) (drill 1.0414) (layers "*.Cu" "*.Mask") (remove_unused_layers no)
   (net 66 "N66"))
  (pad "17" thru_hole circle (at 22.063999 0 270) (size 1.5494 1.5494) (drill 1.0414) (layers "*.Cu" "*.Mask") (remove_unused_layers no)
   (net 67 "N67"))
  (pad "18" thru_hole circle (at 23.443001 2.839999 270) (size 1.5494 1.5494) (drill 1.0414) (layers "*.Cu" "*.Mask")
   (remove_unused_layers no) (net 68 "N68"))
  (pad "19" thru_hole circle (at 24.822 0 270) (size 1.5494 1.5494) (drill 1.0414) (layers "*.Cu" "*.Mask") (remove_unused_layers no)
   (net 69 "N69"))
  (pad "20" thru_hole circle (at 26.201002 2.839999 270) (size 1.5494 1.5494) (drill 1.0414) (layers "*.Cu" "*.Mask")
   (remove_unused_layers no) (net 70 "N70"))
  (pad "21" thru_hole circle (at 27.580001 0 270) (size 1.5494 1.5494) (drill 1.0414) (layers "*.Cu" "*.Mask") (remove_unused_layers no)
   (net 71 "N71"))
  (pad "22" thru_hole circle (at 28.959 2.839999 270) (size 1.5494 1.5494) (drill 1.0414) (layers "*.Cu" "*.Mask") (remove_unused_layers no)
   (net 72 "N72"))
  (pad "23" thru_hole circle (at 30.338001 0 270) (size 1.5494 1.5494) (drill 1.0414) (layers "*.Cu" "*.Mask") (remove_unused_layers no)
   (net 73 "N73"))
  (pad "24" thru_hole circle (at 31.717 2.839999 270) (size 1.5494 1.5494) (drill 1.0414) (layers "*.Cu" "*.Mask") (remove_unused_layers no)
   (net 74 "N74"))
  (pad "25" thru_hole circle (at 33.096002 0 270) (size 1.5494 1.5494) (drill 1.0414) (layers "*.Cu" "*.Mask") (remove_unused_layers no)
   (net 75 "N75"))
  (pad "26" thru_hole circle (at -6.972006 1.42 270) (size 3.7592 3.7592) (drill 3.2512) (layers "*.Cu" "*.Mask") (remove_unused_layers no))
  (pad "27" thru_hole circle (at 40.068007 1.42 270) (size 3.7592 3.7592) (drill 3.2512) (layers "*.Cu" "*.Mask") (remove_unused_layers no)))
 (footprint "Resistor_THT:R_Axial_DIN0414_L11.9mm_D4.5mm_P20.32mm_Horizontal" (layer "F.Cu") (at 62.68 52.5)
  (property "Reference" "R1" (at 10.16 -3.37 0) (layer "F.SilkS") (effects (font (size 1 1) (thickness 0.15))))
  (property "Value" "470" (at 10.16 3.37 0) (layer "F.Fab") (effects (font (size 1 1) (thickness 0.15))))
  (fp_line (start 1.44 0) (end 4.09 0) (stroke (width 0.12) (type solid)) (layer "F.SilkS"))
  (fp_line (start 4.09 -2.37) (end 4.09 2.37) (stroke (width 0.12) (type solid)) (layer "F.SilkS"))
  (fp_line (start 4.09 2.37) (end 16.23 2.37) (stroke (width 0.12) (type solid)) (layer "F.SilkS"))
  (fp_line (start 16.23 -2.37) (end 4.09 -2.37) (stroke (width 0.12) (type solid)) (layer "F.SilkS"))
  (fp_line (start 16.23 2.37) (end 16.23 -2.37) (stroke (width 0.12) (type solid)) (layer "F.SilkS"))
  (fp_line (start 18.88 0) (end 16.23 0) (stroke (width 0.12) (type solid)) (layer "F.SilkS"))
  (pad "1" thru_hole circle (at 0 0) (size 2.4 2.4) (drill 1.2) (layers "*.Cu" "*.Mask") (remove_unused_layers no) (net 1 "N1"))
  (pad "2" thru_hole oval (at 20.32 0) (size 2.4 2.4) (drill 1.2) (layers "*.Cu" "*.Mask") (remove_unused_layers no) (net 63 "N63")))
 (gr_rect (start 123.5 20.5) (end 222.5 150.5) (stroke (width 0.05) (type default)) (fill none) (layer "Edge.Cuts"))
 (segment (start 63 52.82) (end 62.68 52.5) (width 0.2) (layer "F.Cu") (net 1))
 (segment (start 63 67) (end 63 52.82) (width 0.2) (layer "F.Cu") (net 1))
 (segment (start 81.25 66.825) (end 65.715 66.825) (width 0.2) (layer "F.Cu") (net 2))
 (segment (start 65.715 66.825) (end 63 69.54) (width 0.2) (layer "F.Cu") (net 2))
 (segment (start 83 52.5) (end 83 66.035) (width 0.2) (layer "F.Cu") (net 63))
 (segment (start 83 66.035) (end 83.79 66.825) (width 0.2) (layer "F.Cu") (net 63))
 (segment (start 152.461 42.177997) (end 153.839999 40.798998) (width 0.2) (layer "B.Cu") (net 4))
 (segment (start 184.636998 43.556998) (end 202 60.92) (width 0.2) (layer "B.Cu") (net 4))
 (segment (start 202 62.19) (end 202 66) (width 0.2) (layer "B.Cu") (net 4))
 (segment (start 153.839999 43.556998) (end 153.839999 40.798998) (width 0.2) (layer "B.Cu") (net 4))
 (segment (start 153.839999 43.556998) (end 184.636998 43.556998) (width 0.2) (layer "B.Cu") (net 4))
 (segment (start 151 42.177997) (end 152.461 42.177997) (width 0.2) (layer "B.Cu") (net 4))
 (segment (start 202 60.92) (end 202 62.19) (width 0.2) (layer "B.Cu") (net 4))
 (segment (start 151 44.935997) (end 152.460997 44.935997) (width 0.2) (layer "B.Cu") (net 10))
 (segment (start 182.051999 39.724298) (end 202.965 60.637299) (width 0.2) (layer "B.Cu") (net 10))
 (segment (start 202.965 66.305) (end 202 67.27) (width 0.2) (layer "B.Cu") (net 10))
 (segment (start 151.933843 39.724298) (end 182.051999 39.724298) (width 0.2) (layer "B.Cu") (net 10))
 (segment (start 149.9253 41.732841) (end 151.933843 39.724298) (width 0.2) (layer "B.Cu") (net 10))
 (segment (start 152.460997 44.935997) (end 153.839999 46.314999) (width 0.2) (layer "B.Cu") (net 10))
 (segment (start 153.839999 46.314999) (end 152.744408 46.314999) (width 0.2) (layer "B.Cu") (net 10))
 (segment (start 152.744408 46.314999) (end 149.9253 43.495891) (width 0.2) (layer "B.Cu") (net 10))
 (segment (start 202 67.27) (end 202 72.35) (width 0.2) (layer "B.Cu") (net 10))
 (segment (start 149.9253 43.495891) (end 149.9253 41.732841) (width 0.2) (layer "B.Cu") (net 10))
 (segment (start 202.965 60.637299) (end 202.965 66.305) (width 0.2) (layer "B.Cu") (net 10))
 (segment (start 151 47.693998) (end 186.233998 47.693998) (width 0.2) (layer "F.Cu") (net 3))
 (segment (start 186.233998 47.693998) (end 199.46 60.92) (width 0.2) (layer "F.Cu") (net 3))
 (segment (start 179.992997 49.072997) (end 199.46 68.54) (width 0.2) (layer "F.Cu") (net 11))
 (segment (start 153.839999 49.072997) (end 179.992997 49.072997) (width 0.2) (layer "F.Cu") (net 11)))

